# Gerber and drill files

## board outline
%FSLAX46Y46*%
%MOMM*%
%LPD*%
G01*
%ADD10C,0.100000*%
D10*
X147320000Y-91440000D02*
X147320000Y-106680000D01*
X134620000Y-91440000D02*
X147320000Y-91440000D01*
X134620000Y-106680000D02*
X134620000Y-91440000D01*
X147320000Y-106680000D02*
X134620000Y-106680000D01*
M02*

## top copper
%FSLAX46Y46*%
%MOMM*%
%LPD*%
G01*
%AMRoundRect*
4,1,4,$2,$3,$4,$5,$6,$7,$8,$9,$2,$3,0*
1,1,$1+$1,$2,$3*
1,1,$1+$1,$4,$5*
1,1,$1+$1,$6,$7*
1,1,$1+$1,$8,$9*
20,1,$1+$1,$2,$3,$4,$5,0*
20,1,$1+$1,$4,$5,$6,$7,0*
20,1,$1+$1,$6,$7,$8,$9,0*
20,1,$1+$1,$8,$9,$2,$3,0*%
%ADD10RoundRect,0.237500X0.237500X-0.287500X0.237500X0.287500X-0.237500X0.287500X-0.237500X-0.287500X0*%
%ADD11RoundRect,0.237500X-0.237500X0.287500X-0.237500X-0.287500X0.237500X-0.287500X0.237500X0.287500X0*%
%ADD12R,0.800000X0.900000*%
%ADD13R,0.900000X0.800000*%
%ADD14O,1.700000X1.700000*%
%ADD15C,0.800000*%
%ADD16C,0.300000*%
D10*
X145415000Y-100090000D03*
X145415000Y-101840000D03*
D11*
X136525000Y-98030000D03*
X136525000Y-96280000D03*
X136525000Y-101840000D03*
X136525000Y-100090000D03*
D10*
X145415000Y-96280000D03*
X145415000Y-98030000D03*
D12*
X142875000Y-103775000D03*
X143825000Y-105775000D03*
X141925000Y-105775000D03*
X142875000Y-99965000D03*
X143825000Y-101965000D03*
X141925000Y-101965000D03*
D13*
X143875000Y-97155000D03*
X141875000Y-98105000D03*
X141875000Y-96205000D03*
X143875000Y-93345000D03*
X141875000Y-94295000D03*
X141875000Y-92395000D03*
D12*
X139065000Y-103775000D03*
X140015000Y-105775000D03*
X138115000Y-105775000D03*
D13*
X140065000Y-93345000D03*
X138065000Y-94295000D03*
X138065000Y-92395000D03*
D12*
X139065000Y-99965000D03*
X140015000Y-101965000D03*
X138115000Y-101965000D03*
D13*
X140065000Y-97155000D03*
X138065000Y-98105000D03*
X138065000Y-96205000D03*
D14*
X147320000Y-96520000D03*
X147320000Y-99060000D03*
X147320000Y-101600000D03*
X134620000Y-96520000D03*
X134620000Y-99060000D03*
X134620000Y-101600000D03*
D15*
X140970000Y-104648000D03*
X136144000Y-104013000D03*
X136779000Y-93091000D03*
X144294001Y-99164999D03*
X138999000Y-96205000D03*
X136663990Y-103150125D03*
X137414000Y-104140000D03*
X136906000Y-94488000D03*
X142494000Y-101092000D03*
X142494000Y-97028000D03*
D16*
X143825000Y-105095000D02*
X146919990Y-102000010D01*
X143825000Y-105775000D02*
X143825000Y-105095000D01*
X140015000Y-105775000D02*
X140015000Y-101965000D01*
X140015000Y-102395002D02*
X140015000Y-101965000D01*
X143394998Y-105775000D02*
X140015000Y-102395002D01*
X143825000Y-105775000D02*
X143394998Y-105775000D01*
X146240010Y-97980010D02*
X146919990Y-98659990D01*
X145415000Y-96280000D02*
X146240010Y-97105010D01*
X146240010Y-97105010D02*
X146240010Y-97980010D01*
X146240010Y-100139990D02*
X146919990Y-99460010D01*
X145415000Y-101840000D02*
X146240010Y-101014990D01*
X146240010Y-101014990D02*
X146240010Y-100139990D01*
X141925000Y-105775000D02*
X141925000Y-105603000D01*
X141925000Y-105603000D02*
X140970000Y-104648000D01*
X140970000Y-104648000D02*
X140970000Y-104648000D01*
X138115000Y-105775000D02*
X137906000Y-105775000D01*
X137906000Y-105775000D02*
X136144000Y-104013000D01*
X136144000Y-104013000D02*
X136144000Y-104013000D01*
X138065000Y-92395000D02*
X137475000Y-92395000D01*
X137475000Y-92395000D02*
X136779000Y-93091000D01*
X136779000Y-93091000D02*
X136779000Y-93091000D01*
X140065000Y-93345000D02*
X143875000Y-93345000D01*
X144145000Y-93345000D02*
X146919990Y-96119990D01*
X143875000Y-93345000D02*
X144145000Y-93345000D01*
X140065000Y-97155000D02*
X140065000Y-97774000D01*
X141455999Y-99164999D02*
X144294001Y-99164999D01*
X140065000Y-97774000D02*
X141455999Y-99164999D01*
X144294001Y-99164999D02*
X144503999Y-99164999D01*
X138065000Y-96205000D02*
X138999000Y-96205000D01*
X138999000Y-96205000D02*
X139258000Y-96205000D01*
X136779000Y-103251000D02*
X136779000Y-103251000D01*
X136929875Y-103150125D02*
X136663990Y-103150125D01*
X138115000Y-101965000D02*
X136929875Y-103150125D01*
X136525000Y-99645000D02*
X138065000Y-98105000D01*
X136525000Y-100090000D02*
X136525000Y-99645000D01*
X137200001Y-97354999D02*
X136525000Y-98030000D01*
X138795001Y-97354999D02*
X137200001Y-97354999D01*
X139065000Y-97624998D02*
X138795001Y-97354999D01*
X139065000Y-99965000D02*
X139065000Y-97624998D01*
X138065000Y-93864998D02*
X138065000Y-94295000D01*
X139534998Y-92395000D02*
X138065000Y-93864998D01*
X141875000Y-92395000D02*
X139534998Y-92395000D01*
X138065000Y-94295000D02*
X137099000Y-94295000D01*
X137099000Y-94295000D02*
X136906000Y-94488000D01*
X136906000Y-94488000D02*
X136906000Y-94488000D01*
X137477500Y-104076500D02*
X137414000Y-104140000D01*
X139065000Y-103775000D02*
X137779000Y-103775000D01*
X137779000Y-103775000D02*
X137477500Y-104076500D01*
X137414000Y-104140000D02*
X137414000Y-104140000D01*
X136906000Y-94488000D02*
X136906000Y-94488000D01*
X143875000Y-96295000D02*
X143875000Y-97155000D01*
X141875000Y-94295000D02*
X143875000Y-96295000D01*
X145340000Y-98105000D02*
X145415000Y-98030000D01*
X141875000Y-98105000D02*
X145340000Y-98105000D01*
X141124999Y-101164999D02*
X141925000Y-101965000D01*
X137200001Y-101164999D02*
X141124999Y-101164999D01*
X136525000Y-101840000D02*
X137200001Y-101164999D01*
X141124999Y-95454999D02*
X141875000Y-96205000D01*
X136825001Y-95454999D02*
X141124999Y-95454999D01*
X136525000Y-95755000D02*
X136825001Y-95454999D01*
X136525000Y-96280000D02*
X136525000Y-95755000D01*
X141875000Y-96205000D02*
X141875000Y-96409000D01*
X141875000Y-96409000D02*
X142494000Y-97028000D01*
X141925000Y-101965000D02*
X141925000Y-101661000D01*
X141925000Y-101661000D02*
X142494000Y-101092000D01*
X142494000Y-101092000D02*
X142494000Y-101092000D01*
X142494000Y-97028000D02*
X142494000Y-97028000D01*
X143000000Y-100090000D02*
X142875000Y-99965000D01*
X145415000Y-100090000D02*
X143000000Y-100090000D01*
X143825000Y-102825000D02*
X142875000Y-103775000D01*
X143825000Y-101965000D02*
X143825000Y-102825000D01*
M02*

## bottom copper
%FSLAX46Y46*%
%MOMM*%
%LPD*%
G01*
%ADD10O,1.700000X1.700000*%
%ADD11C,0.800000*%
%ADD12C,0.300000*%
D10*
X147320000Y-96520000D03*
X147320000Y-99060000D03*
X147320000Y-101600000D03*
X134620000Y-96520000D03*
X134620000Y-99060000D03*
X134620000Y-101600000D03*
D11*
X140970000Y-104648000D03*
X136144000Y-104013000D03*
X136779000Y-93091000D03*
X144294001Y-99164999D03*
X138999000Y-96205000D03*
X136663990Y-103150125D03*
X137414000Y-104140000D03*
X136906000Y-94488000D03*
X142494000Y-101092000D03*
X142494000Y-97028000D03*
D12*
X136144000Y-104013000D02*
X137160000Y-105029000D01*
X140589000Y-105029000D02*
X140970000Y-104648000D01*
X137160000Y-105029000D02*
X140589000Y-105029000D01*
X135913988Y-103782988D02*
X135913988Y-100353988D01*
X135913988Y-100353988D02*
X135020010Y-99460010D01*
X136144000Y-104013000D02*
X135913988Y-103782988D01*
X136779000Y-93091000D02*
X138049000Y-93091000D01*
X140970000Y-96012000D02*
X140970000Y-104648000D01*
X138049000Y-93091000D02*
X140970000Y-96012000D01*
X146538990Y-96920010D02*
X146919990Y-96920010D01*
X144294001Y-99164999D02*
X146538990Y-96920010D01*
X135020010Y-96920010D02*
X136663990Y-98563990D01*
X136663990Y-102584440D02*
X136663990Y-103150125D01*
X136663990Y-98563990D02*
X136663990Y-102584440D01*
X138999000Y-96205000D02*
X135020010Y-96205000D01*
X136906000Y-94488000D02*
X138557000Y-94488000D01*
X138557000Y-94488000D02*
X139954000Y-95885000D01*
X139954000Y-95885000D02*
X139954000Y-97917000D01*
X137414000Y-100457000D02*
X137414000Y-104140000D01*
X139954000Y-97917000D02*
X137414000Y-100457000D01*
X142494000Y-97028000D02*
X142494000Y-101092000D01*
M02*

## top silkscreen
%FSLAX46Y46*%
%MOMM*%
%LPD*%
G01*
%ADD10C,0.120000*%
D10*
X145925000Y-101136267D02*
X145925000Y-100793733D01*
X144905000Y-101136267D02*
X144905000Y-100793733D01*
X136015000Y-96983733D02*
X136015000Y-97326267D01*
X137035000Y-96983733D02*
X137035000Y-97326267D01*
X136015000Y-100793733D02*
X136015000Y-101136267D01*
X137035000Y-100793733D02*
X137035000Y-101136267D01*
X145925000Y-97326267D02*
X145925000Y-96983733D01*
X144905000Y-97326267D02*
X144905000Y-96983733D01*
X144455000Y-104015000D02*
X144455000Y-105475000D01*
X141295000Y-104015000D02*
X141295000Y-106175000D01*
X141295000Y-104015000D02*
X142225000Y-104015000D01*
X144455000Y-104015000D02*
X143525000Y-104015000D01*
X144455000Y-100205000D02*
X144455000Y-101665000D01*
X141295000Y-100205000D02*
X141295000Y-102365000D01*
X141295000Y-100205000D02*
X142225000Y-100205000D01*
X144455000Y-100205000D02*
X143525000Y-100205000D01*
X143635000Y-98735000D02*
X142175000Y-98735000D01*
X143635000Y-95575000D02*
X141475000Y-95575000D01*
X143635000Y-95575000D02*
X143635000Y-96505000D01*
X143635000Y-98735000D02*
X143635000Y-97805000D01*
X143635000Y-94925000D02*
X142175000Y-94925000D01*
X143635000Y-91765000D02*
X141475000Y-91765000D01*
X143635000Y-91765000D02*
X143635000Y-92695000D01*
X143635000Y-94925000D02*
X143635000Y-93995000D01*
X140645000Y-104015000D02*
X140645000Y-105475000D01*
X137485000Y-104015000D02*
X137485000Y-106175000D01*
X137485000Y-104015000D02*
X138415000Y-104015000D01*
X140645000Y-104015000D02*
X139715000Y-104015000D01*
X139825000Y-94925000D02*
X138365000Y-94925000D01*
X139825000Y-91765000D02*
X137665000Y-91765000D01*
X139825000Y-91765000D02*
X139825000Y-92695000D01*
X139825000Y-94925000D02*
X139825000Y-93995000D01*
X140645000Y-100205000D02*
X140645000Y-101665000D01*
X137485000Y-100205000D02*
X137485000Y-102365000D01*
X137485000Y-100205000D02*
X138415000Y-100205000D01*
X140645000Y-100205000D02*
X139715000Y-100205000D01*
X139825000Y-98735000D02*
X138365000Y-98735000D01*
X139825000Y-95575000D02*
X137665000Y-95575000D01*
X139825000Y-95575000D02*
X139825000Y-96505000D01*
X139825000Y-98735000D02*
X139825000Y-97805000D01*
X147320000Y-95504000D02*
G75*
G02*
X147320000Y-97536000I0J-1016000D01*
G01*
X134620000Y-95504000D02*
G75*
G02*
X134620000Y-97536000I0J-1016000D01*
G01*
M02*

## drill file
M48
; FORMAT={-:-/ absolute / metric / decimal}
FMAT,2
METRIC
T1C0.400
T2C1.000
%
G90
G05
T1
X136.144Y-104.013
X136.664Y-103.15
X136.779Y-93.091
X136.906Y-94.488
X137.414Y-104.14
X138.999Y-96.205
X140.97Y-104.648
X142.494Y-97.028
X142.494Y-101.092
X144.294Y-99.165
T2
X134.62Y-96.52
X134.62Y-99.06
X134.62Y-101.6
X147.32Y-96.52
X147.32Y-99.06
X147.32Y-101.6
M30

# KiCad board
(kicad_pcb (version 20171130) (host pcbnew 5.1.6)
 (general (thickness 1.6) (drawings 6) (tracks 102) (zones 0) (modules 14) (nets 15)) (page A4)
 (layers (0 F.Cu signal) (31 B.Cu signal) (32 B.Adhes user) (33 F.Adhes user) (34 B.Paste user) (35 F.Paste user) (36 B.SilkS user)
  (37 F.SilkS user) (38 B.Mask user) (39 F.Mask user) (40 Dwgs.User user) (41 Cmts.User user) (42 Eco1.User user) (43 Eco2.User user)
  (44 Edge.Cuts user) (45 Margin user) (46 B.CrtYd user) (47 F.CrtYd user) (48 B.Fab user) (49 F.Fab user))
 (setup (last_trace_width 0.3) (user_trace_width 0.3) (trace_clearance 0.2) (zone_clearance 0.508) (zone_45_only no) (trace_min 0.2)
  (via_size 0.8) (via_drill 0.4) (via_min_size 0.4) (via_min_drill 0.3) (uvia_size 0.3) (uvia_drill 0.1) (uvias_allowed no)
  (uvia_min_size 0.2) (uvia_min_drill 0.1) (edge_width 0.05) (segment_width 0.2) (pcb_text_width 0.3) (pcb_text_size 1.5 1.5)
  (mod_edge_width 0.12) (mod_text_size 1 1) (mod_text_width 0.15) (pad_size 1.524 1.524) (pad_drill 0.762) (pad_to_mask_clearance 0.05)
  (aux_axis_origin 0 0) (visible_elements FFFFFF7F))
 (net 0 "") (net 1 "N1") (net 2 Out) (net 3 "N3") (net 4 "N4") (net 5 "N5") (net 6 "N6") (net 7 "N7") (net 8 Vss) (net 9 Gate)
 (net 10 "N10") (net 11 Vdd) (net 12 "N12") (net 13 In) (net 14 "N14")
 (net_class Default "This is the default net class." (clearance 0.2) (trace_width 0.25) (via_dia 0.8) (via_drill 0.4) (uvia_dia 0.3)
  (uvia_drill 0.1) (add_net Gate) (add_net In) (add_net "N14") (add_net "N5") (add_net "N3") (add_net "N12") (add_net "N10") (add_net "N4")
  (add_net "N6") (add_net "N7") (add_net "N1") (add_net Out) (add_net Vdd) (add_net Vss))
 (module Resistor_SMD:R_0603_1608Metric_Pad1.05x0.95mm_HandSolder (layer F.Cu) (at 145.415 100.965 90)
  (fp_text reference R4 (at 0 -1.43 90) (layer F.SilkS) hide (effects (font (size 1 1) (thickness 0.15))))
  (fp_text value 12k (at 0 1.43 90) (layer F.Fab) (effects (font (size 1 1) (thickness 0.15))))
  (fp_line (start -0.171267 0.51) (end 0.171267 0.51) (layer F.SilkS) (width 0.12))
  (fp_line (start -0.171267 -0.51) (end 0.171267 -0.51) (layer F.SilkS) (width 0.12))
  (pad 2 smd roundrect (at 0.875 0 90) (size 1.05 0.95) (layers F.Cu F.Paste F.Mask) (roundrect_rratio 0.25) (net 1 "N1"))
  (pad 1 smd roundrect (at -0.875 0 90) (size 1.05 0.95) (layers F.Cu F.Paste F.Mask) (roundrect_rratio 0.25) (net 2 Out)))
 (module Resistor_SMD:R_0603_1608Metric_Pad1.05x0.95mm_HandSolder (layer F.Cu) (at 136.525 97.155 270)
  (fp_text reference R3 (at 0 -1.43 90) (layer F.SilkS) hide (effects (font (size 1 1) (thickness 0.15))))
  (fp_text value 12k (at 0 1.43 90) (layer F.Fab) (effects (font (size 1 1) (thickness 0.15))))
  (fp_line (start -0.171267 0.51) (end 0.171267 0.51) (layer F.SilkS) (width 0.12))
  (fp_line (start -0.171267 -0.51) (end 0.171267 -0.51) (layer F.SilkS) (width 0.12))
  (pad 2 smd roundrect (at 0.875 0 270) (size 1.05 0.95) (layers F.Cu F.Paste F.Mask) (roundrect_rratio 0.25) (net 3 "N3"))
  (pad 1 smd roundrect (at -0.875 0 270) (size 1.05 0.95) (layers F.Cu F.Paste F.Mask) (roundrect_rratio 0.25) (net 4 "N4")))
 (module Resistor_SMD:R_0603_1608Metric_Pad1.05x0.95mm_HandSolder (layer F.Cu) (at 136.525 100.965 270)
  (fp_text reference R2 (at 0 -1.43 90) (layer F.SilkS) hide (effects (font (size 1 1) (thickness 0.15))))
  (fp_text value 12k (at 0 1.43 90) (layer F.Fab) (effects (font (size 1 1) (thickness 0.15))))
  (fp_line (start -0.171267 0.51) (end 0.171267 0.51) (layer F.SilkS) (width 0.12))
  (fp_line (start -0.171267 -0.51) (end 0.171267 -0.51) (layer F.SilkS) (width 0.12))
  (pad 2 smd roundrect (at 0.875 0 270) (size 1.05 0.95) (layers F.Cu F.Paste F.Mask) (roundrect_rratio 0.25) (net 4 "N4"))
  (pad 1 smd roundrect (at -0.875 0 270) (size 1.05 0.95) (layers F.Cu F.Paste F.Mask) (roundrect_rratio 0.25) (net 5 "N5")))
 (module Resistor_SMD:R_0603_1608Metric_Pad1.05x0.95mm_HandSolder (layer F.Cu) (at 145.415 97.155 90)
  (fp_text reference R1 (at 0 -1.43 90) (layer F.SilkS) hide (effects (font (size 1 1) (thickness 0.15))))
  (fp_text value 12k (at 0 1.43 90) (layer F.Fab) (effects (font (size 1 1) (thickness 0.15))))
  (fp_line (start -0.171267 0.51) (end 0.171267 0.51) (layer F.SilkS) (width 0.12))
  (fp_line (start -0.171267 -0.51) (end 0.171267 -0.51) (layer F.SilkS) (width 0.12))
  (pad 2 smd roundrect (at 0.875 0 90) (size 1.05 0.95) (layers F.Cu F.Paste F.Mask) (roundrect_rratio 0.25) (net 2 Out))
  (pad 1 smd roundrect (at -0.875 0 90) (size 1.05 0.95) (layers F.Cu F.Paste F.Mask) (roundrect_rratio 0.25) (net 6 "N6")))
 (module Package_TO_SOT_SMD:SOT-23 (layer F.Cu) (at 142.875 104.775 90)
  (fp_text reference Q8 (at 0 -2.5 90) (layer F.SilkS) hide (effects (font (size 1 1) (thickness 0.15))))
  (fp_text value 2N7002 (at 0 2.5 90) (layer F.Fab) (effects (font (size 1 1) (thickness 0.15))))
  (fp_line (start 0.76 1.58) (end -0.7 1.58) (layer F.SilkS) (width 0.12))
  (fp_line (start 0.76 -1.58) (end -1.4 -1.58) (layer F.SilkS) (width 0.12))
  (fp_line (start 0.76 -1.58) (end 0.76 -0.65) (layer F.SilkS) (width 0.12))
  (fp_line (start 0.76 1.58) (end 0.76 0.65) (layer F.SilkS) (width 0.12))
  (pad 3 smd rect (at 1 0 90) (size 0.9 0.8) (layers F.Cu F.Paste F.Mask) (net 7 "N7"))
  (pad 2 smd rect (at -1 0.95 90) (size 0.9 0.8) (layers F.Cu F.Paste F.Mask) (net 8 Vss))
  (pad 1 smd rect (at -1 -0.95 90) (size 0.9 0.8) (layers F.Cu F.Paste F.Mask) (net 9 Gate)))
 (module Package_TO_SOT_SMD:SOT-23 (layer F.Cu) (at 142.875 100.965 90)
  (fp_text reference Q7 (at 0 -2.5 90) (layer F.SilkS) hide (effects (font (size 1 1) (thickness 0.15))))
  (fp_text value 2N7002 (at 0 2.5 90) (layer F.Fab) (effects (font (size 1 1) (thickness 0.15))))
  (fp_line (start 0.76 1.58) (end -0.7 1.58) (layer F.SilkS) (width 0.12))
  (fp_line (start 0.76 -1.58) (end -1.4 -1.58) (layer F.SilkS) (width 0.12))
  (fp_line (start 0.76 -1.58) (end 0.76 -0.65) (layer F.SilkS) (width 0.12))
  (fp_line (start 0.76 1.58) (end 0.76 0.65) (layer F.SilkS) (width 0.12))
  (pad 3 smd rect (at 1 0 90) (size 0.9 0.8) (layers F.Cu F.Paste F.Mask) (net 1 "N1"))
  (pad 2 smd rect (at -1 0.95 90) (size 0.9 0.8) (layers F.Cu F.Paste F.Mask) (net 7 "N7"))
  (pad 1 smd rect (at -1 -0.95 90) (size 0.9 0.8) (layers F.Cu F.Paste F.Mask) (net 4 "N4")))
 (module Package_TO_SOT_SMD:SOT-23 (layer F.Cu) (at 142.875 97.155)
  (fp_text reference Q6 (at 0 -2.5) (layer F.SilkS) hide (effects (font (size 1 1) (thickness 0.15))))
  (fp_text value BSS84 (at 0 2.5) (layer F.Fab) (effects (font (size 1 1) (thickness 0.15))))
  (fp_line (start 0.76 1.58) (end -0.7 1.58) (layer F.SilkS) (width 0.12))
  (fp_line (start 0.76 -1.58) (end -1.4 -1.58) (layer F.SilkS) (width 0.12))
  (fp_line (start 0.76 -1.58) (end 0.76 -0.65) (layer F.SilkS) (width 0.12))
  (fp_line (start 0.76 1.58) (end 0.76 0.65) (layer F.SilkS) (width 0.12))
  (pad 3 smd rect (at 1 0) (size 0.9 0.8) (layers F.Cu F.Paste F.Mask) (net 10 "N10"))
  (pad 2 smd rect (at -1 0.95) (size 0.9 0.8) (layers F.Cu F.Paste F.Mask) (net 6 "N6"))
  (pad 1 smd rect (at -1 -0.95) (size 0.9 0.8) (layers F.Cu F.Paste F.Mask) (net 4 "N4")))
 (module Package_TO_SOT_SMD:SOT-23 (layer F.Cu) (at 142.875 93.345)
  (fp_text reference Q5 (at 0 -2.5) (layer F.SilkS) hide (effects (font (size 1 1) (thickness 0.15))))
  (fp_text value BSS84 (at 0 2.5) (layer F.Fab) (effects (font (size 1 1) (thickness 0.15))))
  (fp_line (start 0.76 1.58) (end -0.7 1.58) (layer F.SilkS) (width 0.12))
  (fp_line (start 0.76 -1.58) (end -1.4 -1.58) (layer F.SilkS) (width 0.12))
  (fp_line (start 0.76 -1.58) (end 0.76 -0.65) (layer F.SilkS) (width 0.12))
  (fp_line (start 0.76 1.58) (end 0.76 0.65) (layer F.SilkS) (width 0.12))
  (pad 3 smd rect (at 1 0) (size 0.9 0.8) (layers F.Cu F.Paste F.Mask) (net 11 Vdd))
  (pad 2 smd rect (at -1 0.95) (size 0.9 0.8) (layers F.Cu F.Paste F.Mask) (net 10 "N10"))
  (pad 1 smd rect (at -1 -0.95) (size 0.9 0.8) (layers F.Cu F.Paste F.Mask) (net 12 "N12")))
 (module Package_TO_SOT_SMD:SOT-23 (layer F.Cu) (at 139.065 104.775 90)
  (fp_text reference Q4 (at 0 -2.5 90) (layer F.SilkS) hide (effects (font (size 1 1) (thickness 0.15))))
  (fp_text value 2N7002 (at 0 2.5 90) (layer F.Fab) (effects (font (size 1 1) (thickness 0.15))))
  (fp_line (start 0.76 1.58) (end -0.7 1.58) (layer F.SilkS) (width 0.12))
  (fp_line (start 0.76 -1.58) (end -1.4 -1.58) (layer F.SilkS) (width 0.12))
  (fp_line (start 0.76 -1.58) (end 0.76 -0.65) (layer F.SilkS) (width 0.12))
  (fp_line (start 0.76 1.58) (end 0.76 0.65) (layer F.SilkS) (width 0.12))
  (pad 3 smd rect (at 1 0 90) (size 0.9 0.8) (layers F.Cu F.Paste F.Mask) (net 12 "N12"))
  (pad 2 smd rect (at -1 0.95 90) (size 0.9 0.8) (layers F.Cu F.Paste F.Mask) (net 8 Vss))
  (pad 1 smd rect (at -1 -0.95 90) (size 0.9 0.8) (layers F.Cu F.Paste F.Mask) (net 9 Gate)))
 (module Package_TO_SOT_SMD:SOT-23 (layer F.Cu) (at 139.065 93.345)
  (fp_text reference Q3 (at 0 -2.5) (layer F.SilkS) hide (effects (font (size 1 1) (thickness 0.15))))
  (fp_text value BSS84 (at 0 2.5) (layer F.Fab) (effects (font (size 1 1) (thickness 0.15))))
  (fp_line (start 0.76 1.58) (end -0.7 1.58) (layer F.SilkS) (width 0.12))
  (fp_line (start 0.76 -1.58) (end -1.4 -1.58) (layer F.SilkS) (width 0.12))
  (fp_line (start 0.76 -1.58) (end 0.76 -0.65) (layer F.SilkS) (width 0.12))
  (fp_line (start 0.76 1.58) (end 0.76 0.65) (layer F.SilkS) (width 0.12))
  (pad 3 smd rect (at 1 0) (size 0.9 0.8) (layers F.Cu F.Paste F.Mask) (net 11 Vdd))
  (pad 2 smd rect (at -1 0.95) (size 0.9 0.8) (layers F.Cu F.Paste F.Mask) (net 12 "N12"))
  (pad 1 smd rect (at -1 -0.95) (size 0.9 0.8) (layers F.Cu F.Paste F.Mask) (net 9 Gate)))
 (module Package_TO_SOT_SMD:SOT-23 (layer F.Cu) (at 139.065 100.965 90)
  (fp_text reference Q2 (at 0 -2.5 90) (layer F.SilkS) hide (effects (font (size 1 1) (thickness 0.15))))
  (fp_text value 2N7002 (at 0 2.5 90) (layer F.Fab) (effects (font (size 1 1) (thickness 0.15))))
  (fp_line (start 0.76 1.58) (end -0.7 1.58) (layer F.SilkS) (width 0.12))
  (fp_line (start 0.76 -1.58) (end -1.4 -1.58) (layer F.SilkS) (width 0.12))
  (fp_line (start 0.76 -1.58) (end 0.76 -0.65) (layer F.SilkS) (width 0.12))
  (fp_line (start 0.76 1.58) (end 0.76 0.65) (layer F.SilkS) (width 0.12))
  (pad 3 smd rect (at 1 0 90) (size 0.9 0.8) (layers F.Cu F.Paste F.Mask) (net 3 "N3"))
  (pad 2 smd rect (at -1 0.95 90) (size 0.9 0.8) (layers F.Cu F.Paste F.Mask) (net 8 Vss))
  (pad 1 smd rect (at -1 -0.95 90) (size 0.9 0.8) (layers F.Cu F.Paste F.Mask) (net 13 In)))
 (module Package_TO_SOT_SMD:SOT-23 (layer F.Cu) (at 139.065 97.155)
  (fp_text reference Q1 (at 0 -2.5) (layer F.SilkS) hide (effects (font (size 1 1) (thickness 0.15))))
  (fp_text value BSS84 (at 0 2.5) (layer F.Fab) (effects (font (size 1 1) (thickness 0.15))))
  (fp_line (start 0.76 1.58) (end -0.7 1.58) (layer F.SilkS) (width 0.12))
  (fp_line (start 0.76 -1.58) (end -1.4 -1.58) (layer F.SilkS) (width 0.12))
  (fp_line (start 0.76 -1.58) (end 0.76 -0.65) (layer F.SilkS) (width 0.12))
  (fp_line (start 0.76 1.58) (end 0.76 0.65) (layer F.SilkS) (width 0.12))
  (pad 3 smd rect (at 1 0) (size 0.9 0.8) (layers F.Cu F.Paste F.Mask) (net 11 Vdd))
  (pad 2 smd rect (at -1 0.95) (size 0.9 0.8) (layers F.Cu F.Paste F.Mask) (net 5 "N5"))
  (pad 1 smd rect (at -1 -0.95) (size 0.9 0.8) (layers F.Cu F.Paste F.Mask) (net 13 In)))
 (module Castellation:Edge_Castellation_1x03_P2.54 (layer F.Cu) (at 147.32 96.52)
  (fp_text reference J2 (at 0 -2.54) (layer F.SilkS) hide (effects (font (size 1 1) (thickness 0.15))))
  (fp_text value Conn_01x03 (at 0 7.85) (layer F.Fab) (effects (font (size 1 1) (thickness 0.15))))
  (fp_arc (start 0 0) (end 0 1.016) (angle -180) (layer F.SilkS) (width 0.12))
  (pad 1 thru_hole oval (at 0 0) (size 1.7 1.7) (drill 1) (layers *.Cu *.Mask) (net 11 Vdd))
  (pad 2 thru_hole oval (at 0 2.54) (size 1.7 1.7) (drill 1) (layers *.Cu *.Mask) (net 2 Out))
  (pad 3 thru_hole oval (at 0 5.08) (size 1.7 1.7) (drill 1) (layers *.Cu *.Mask) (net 8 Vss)))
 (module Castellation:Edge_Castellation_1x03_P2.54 (layer F.Cu) (at 134.62 96.52)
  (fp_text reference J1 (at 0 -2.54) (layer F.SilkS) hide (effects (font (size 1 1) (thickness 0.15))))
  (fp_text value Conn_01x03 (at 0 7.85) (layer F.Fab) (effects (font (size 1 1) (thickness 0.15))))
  (fp_arc (start 0 0) (end 0 1.016) (angle -180) (layer F.SilkS) (width 0.12))
  (pad 1 thru_hole oval (at 0 0) (size 1.7 1.7) (drill 1) (layers *.Cu *.Mask) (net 13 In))
  (pad 2 thru_hole oval (at 0 2.54) (size 1.7 1.7) (drill 1) (layers *.Cu *.Mask) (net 9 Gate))
  (pad 3 thru_hole oval (at 0 5.08) (size 1.7 1.7) (drill 1) (layers *.Cu *.Mask) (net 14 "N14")))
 (gr_line (start 147.32 91.44) (end 147.32 106.68) (layer Edge.Cuts) (width 0.1))
 (gr_line (start 134.62 91.44) (end 147.32 91.44) (layer Edge.Cuts) (width 0.1))
 (gr_line (start 134.62 106.68) (end 134.62 91.44) (layer Edge.Cuts) (width 0.1))
 (gr_line (start 147.32 106.68) (end 134.62 106.68) (layer Edge.Cuts) (width 0.1))
 (segment (start 143.825 105.095) (end 146.91999 102.00001) (width 0.3) (layer F.Cu) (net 8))
 (segment (start 143.825 105.775) (end 143.825 105.095) (width 0.3) (layer F.Cu) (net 8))
 (segment (start 140.015 105.775) (end 140.015 101.965) (width 0.3) (layer F.Cu) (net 8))
 (segment (start 140.015 102.395002) (end 140.015 101.965) (width 0.3) (layer F.Cu) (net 8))
 (segment (start 143.394998 105.775) (end 140.015 102.395002) (width 0.3) (layer F.Cu) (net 8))
 (segment (start 143.825 105.775) (end 143.394998 105.775) (width 0.3) (layer F.Cu) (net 8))
 (segment (start 146.24001 97.98001) (end 146.91999 98.65999) (width 0.3) (layer F.Cu) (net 2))
 (segment (start 145.415 96.28) (end 146.24001 97.10501) (width 0.3) (layer F.Cu) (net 2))
 (segment (start 146.24001 97.10501) (end 146.24001 97.98001) (width 0.3) (layer F.Cu) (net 2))
 (segment (start 146.24001 100.13999) (end 146.91999 99.46001) (width 0.3) (layer F.Cu) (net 2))
 (segment (start 145.415 101.84) (end 146.24001 101.01499) (width 0.3) (layer F.Cu) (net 2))
 (segment (start 146.24001 101.01499) (end 146.24001 100.13999) (width 0.3) (layer F.Cu) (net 2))
 (segment (start 141.925 105.775) (end 141.925 105.603) (width 0.3) (layer F.Cu) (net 9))
 (segment (start 141.925 105.603) (end 140.97 104.648) (width 0.3) (layer F.Cu) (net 9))
 (segment (start 140.97 104.648) (end 140.97 104.648) (width 0.3) (layer F.Cu) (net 9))
 (via (at 140.97 104.648) (size 0.8) (drill 0.4) (layers F.Cu B.Cu) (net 9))
 (segment (start 138.115 105.775) (end 137.906 105.775) (width 0.3) (layer F.Cu) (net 9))
 (segment (start 137.906 105.775) (end 136.144 104.013) (width 0.3) (layer F.Cu) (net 9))
 (segment (start 136.144 104.013) (end 136.144 104.013) (width 0.3) (layer F.Cu) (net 9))
 (via (at 136.144 104.013) (size 0.8) (drill 0.4) (layers F.Cu B.Cu) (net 9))
 (segment (start 138.065 92.395) (end 137.475 92.395) (width 0.3) (layer F.Cu) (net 9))
 (segment (start 137.475 92.395) (end 136.779 93.091) (width 0.3) (layer F.Cu) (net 9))
 (segment (start 136.779 93.091) (end 136.779 93.091) (width 0.3) (layer F.Cu) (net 9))
 (via (at 136.779 93.091) (size 0.8) (drill 0.4) (layers F.Cu B.Cu) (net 9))
 (segment (start 136.144 104.013) (end 137.16 105.029) (width 0.3) (layer B.Cu) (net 9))
 (segment (start 140.589 105.029) (end 140.97 104.648) (width 0.3) (layer B.Cu) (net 9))
 (segment (start 137.16 105.029) (end 140.589 105.029) (width 0.3) (layer B.Cu) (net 9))
 (segment (start 135.913988 103.782988) (end 135.913988 100.353988) (width 0.3) (layer B.Cu) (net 9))
 (segment (start 135.913988 100.353988) (end 135.02001 99.46001) (width 0.3) (layer B.Cu) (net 9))
 (segment (start 136.144 104.013) (end 135.913988 103.782988) (width 0.3) (layer B.Cu) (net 9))
 (segment (start 136.779 93.091) (end 138.049 93.091) (width 0.3) (layer B.Cu) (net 9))
 (segment (start 140.97 96.012) (end 140.97 104.648) (width 0.3) (layer B.Cu) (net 9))
 (segment (start 138.049 93.091) (end 140.97 96.012) (width 0.3) (layer B.Cu) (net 9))
 (segment (start 140.065 93.345) (end 143.875 93.345) (width 0.3) (layer F.Cu) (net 11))
 (segment (start 144.145 93.345) (end 146.91999 96.11999) (width 0.3) (layer F.Cu) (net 11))
 (segment (start 143.875 93.345) (end 144.145 93.345) (width 0.3) (layer F.Cu) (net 11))
 (segment (start 140.065 97.155) (end 140.065 97.774) (width 0.3) (layer F.Cu) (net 11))
 (segment (start 141.455999 99.164999) (end 144.294001 99.164999) (width 0.3) (layer F.Cu) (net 11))
 (segment (start 140.065 97.774) (end 141.455999 99.164999) (width 0.3) (layer F.Cu) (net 11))
 (segment (start 144.294001 99.164999) (end 144.503999 99.164999) (width 0.3) (layer F.Cu) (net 11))
 (via (at 144.294001 99.164999) (size 0.8) (drill 0.4) (layers F.Cu B.Cu) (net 11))
 (segment (start 146.53899 96.92001) (end 146.91999 96.92001) (width 0.3) (layer B.Cu) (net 11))
 (segment (start 144.294001 99.164999) (end 146.53899 96.92001) (width 0.3) (layer B.Cu) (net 11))
 (segment (start 138.065 96.205) (end 138.999 96.205) (width 0.3) (layer F.Cu) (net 13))
 (segment (start 138.999 96.205) (end 139.258 96.205) (width 0.3) (layer F.Cu) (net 13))
 (via (at 138.999 96.205) (size 0.8) (drill 0.4) (layers F.Cu B.Cu) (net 13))
 (segment (start 136.779 103.251) (end 136.779 103.251) (width 0.3) (layer F.Cu) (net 13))
 (segment (start 136.929875 103.150125) (end 136.66399 103.150125) (width 0.3) (layer F.Cu) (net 13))
 (segment (start 135.02001 96.92001) (end 136.66399 98.56399) (width 0.3) (layer B.Cu) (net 13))
 (segment (start 136.66399 102.58444) (end 136.66399 103.150125) (width 0.3) (layer B.Cu) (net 13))
 (via (at 136.66399 103.150125) (size 0.8) (drill 0.4) (layers F.Cu B.Cu) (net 13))
 (segment (start 138.115 101.965) (end 136.929875 103.150125) (width 0.3) (layer F.Cu) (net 13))
 (segment (start 136.66399 98.56399) (end 136.66399 102.58444) (width 0.3) (layer B.Cu) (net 13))
 (segment (start 138.999 96.205) (end 135.02001 96.205) (width 0.3) (layer B.Cu) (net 13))
 (segment (start 136.525 99.645) (end 138.065 98.105) (width 0.3) (layer F.Cu) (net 5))
 (segment (start 136.525 100.09) (end 136.525 99.645) (width 0.3) (layer F.Cu) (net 5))
 (segment (start 137.200001 97.354999) (end 136.525 98.03) (width 0.3) (layer F.Cu) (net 3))
 (segment (start 138.795001 97.354999) (end 137.200001 97.354999) (width 0.3) (layer F.Cu) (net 3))
 (segment (start 139.065 97.624998) (end 138.795001 97.354999) (width 0.3) (layer F.Cu) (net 3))
 (segment (start 139.065 99.965) (end 139.065 97.624998) (width 0.3) (layer F.Cu) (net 3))
 (segment (start 138.065 93.864998) (end 138.065 94.295) (width 0.3) (layer F.Cu) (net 12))
 (segment (start 139.534998 92.395) (end 138.065 93.864998) (width 0.3) (layer F.Cu) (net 12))
 (segment (start 141.875 92.395) (end 139.534998 92.395) (width 0.3) (layer F.Cu) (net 12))
 (segment (start 138.065 94.295) (end 137.099 94.295) (width 0.3) (layer F.Cu) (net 12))
 (segment (start 137.099 94.295) (end 136.906 94.488) (width 0.3) (layer F.Cu) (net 12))
 (segment (start 136.906 94.488) (end 136.906 94.488) (width 0.3) (layer F.Cu) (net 12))
 (segment (start 137.4775 104.0765) (end 137.414 104.14) (width 0.3) (layer F.Cu) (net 12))
 (segment (start 139.065 103.775) (end 137.779 103.775) (width 0.3) (layer F.Cu) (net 12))
 (segment (start 137.779 103.775) (end 137.4775 104.0765) (width 0.3) (layer F.Cu) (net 12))
 (segment (start 137.414 104.14) (end 137.414 104.14) (width 0.3) (layer F.Cu) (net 12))
 (via (at 137.414 104.14) (size 0.8) (drill 0.4) (layers F.Cu B.Cu) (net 12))
 (segment (start 136.906 94.488) (end 136.906 94.488) (width 0.3) (layer F.Cu) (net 12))
 (via (at 136.906 94.488) (size 0.8) (drill 0.4) (layers F.Cu B.Cu) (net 12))
 (segment (start 136.906 94.488) (end 138.557 94.488) (width 0.3) (layer B.Cu) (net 12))
 (segment (start 138.557 94.488) (end 139.954 95.885) (width 0.3) (layer B.Cu) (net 12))
 (segment (start 139.954 95.885) (end 139.954 97.917) (width 0.3) (layer B.Cu) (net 12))
 (segment (start 137.414 100.457) (end 137.414 104.14) (width 0.3) (layer B.Cu) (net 12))
 (segment (start 139.954 97.917) (end 137.414 100.457) (width 0.3) (layer B.Cu) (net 12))
 (segment (start 143.875 96.295) (end 143.875 97.155) (width 0.3) (layer F.Cu) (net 10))
 (segment (start 141.875 94.295) (end 143.875 96.295) (width 0.3) (layer F.Cu) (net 10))
 (segment (start 145.34 98.105) (end 145.415 98.03) (width 0.3) (layer F.Cu) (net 6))
 (segment (start 141.875 98.105) (end 145.34 98.105) (width 0.3) (layer F.Cu) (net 6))
 (segment (start 141.124999 101.164999) (end 141.925 101.965) (width 0.3) (layer F.Cu) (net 4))
 (segment (start 137.200001 101.164999) (end 141.124999 101.164999) (width 0.3) (layer F.Cu) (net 4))
 (segment (start 136.525 101.84) (end 137.200001 101.164999) (width 0.3) (layer F.Cu) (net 4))
 (segment (start 141.124999 95.454999) (end 141.875 96.205) (width 0.3) (layer F.Cu) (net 4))
 (segment (start 136.825001 95.454999) (end 141.124999 95.454999) (width 0.3) (layer F.Cu) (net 4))
 (segment (start 136.525 95.755) (end 136.825001 95.454999) (width 0.3) (layer F.Cu) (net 4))
 (segment (start 136.525 96.28) (end 136.525 95.755) (width 0.3) (layer F.Cu) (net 4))
 (segment (start 141.875 96.205) (end 141.875 96.409) (width 0.3) (layer F.Cu) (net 4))
 (segment (start 141.875 96.409) (end 142.494 97.028) (width 0.3) (layer F.Cu) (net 4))
 (segment (start 141.925 101.965) (end 141.925 101.661) (width 0.3) (layer F.Cu) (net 4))
 (segment (start 141.925 101.661) (end 142.494 101.092) (width 0.3) (layer F.Cu) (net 4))
 (segment (start 142.494 101.092) (end 142.494 101.092) (width 0.3) (layer F.Cu) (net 4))
 (via (at 142.494 101.092) (size 0.8) (drill 0.4) (layers F.Cu B.Cu) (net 4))
 (segment (start 142.494 97.028) (end 142.494 97.028) (width 0.3) (layer F.Cu) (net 4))
 (via (at 142.494 97.028) (size 0.8) (drill 0.4) (layers F.Cu B.Cu) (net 4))
 (segment (start 142.494 97.028) (end 142.494 101.092) (width 0.3) (layer B.Cu) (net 4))
 (segment (start 143 100.09) (end 142.875 99.965) (width 0.3) (layer F.Cu) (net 1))
 (segment (start 145.415 100.09) (end 143 100.09) (width 0.3) (layer F.Cu) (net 1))
 (segment (start 143.825 102.825) (end 142.875 103.775) (width 0.3) (layer F.Cu) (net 7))
 (segment (start 143.825 101.965) (end 143.825 102.825) (width 0.3) (layer F.Cu) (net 7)))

